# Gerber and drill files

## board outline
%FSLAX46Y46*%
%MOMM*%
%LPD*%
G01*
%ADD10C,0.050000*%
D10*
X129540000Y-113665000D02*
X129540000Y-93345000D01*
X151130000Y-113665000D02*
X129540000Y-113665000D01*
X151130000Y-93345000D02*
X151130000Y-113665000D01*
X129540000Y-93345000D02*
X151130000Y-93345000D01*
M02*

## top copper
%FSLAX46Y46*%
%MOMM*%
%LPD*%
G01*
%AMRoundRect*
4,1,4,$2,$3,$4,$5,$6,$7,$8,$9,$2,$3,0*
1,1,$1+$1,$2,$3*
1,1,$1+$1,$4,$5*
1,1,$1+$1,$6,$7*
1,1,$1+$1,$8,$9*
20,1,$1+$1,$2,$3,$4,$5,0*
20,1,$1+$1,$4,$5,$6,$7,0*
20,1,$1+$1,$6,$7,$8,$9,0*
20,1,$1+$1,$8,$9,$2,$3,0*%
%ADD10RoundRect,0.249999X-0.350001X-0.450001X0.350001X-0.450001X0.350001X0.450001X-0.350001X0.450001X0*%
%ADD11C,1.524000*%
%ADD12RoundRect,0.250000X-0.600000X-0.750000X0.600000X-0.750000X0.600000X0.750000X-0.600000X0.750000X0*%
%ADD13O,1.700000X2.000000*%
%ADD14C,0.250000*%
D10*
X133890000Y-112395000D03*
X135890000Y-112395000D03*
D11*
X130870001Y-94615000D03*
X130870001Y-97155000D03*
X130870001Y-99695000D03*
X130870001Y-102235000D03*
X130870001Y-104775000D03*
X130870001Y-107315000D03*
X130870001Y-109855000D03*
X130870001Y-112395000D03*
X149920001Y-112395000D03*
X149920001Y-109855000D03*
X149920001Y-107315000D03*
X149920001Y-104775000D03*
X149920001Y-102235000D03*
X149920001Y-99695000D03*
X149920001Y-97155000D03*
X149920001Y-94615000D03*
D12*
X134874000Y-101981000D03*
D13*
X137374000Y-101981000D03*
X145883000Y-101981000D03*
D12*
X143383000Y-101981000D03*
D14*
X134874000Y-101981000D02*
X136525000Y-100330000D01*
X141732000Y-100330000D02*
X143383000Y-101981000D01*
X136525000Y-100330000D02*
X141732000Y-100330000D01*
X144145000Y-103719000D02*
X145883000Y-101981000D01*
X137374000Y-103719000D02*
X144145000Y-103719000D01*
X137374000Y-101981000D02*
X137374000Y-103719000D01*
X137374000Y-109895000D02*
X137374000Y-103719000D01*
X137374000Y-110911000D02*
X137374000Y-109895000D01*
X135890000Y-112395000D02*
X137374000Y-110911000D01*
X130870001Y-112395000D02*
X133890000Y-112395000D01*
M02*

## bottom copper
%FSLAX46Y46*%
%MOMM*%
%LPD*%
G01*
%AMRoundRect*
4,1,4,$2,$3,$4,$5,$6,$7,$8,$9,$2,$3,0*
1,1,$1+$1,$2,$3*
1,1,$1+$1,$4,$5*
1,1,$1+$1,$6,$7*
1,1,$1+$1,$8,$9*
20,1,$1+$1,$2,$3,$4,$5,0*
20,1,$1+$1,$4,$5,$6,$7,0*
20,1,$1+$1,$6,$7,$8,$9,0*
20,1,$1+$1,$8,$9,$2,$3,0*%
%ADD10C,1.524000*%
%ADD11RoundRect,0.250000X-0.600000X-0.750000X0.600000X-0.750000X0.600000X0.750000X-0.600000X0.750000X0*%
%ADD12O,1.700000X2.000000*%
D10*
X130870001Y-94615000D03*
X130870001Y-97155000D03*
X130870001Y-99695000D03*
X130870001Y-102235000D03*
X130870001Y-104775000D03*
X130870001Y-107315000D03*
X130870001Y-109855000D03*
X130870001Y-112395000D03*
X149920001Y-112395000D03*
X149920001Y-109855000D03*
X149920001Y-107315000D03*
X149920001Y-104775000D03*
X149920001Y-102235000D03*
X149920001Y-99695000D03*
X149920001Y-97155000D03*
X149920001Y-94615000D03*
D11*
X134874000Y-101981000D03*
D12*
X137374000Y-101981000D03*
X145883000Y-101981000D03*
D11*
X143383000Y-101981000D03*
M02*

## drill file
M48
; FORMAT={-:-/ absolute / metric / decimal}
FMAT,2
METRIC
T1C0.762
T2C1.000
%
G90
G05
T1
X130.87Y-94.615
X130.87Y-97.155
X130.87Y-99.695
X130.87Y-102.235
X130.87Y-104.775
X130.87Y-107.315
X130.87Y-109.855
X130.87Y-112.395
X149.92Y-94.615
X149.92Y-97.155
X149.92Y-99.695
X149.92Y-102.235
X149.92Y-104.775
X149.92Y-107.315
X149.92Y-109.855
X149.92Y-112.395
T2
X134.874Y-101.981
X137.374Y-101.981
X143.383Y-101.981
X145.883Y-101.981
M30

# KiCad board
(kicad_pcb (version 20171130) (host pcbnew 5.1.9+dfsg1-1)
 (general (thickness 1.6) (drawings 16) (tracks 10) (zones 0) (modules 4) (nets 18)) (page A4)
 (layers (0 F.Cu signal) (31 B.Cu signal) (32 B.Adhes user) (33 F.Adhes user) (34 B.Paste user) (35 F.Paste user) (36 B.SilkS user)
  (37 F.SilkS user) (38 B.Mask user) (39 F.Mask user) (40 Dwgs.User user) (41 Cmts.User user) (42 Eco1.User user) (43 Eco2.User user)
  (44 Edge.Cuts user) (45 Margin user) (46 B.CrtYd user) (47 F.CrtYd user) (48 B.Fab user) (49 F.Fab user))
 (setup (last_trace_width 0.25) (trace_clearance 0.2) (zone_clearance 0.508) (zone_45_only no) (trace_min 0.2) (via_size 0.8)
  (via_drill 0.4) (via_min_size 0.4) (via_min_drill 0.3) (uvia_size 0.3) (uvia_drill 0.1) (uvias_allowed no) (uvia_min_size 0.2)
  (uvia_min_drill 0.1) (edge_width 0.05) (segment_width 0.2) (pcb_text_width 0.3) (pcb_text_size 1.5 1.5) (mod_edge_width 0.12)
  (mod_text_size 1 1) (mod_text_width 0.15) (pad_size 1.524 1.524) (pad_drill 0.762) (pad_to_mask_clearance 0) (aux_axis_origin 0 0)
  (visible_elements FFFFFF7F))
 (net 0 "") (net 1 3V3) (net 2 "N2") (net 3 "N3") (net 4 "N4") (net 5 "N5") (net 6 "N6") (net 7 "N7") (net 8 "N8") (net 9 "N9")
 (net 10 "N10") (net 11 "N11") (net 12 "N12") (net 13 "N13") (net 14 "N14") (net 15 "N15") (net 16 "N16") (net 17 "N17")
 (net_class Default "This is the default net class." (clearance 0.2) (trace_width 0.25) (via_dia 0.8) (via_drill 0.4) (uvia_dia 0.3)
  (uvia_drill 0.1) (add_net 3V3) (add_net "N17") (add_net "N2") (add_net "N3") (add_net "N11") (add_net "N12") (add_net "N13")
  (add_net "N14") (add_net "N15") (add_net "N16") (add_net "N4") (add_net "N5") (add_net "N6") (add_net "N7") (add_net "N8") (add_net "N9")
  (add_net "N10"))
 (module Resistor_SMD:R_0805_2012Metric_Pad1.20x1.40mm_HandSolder (layer F.Cu) (at 134.89 112.395)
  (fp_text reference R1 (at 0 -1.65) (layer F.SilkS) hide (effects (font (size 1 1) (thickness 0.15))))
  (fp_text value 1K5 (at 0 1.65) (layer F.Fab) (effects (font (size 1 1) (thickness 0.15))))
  (pad 1 smd roundrect (at -1 0) (size 1.2 1.4) (layers F.Cu F.Paste F.Mask) (roundrect_rratio 0.2083325) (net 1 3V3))
  (pad 2 smd roundrect (at 1 0) (size 1.2 1.4) (layers F.Cu F.Paste F.Mask) (roundrect_rratio 0.2083325) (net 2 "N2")))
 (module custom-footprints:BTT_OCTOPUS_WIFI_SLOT (layer F.Cu) (at 143.570001 94.615)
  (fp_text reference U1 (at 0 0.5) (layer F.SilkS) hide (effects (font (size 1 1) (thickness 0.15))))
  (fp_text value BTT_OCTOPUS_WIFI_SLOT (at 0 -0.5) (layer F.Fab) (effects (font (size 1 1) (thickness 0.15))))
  (pad 1 thru_hole circle (at -12.7 0) (size 1.524 1.524) (drill 0.762) (layers *.Cu *.Mask) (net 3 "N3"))
  (pad 2 thru_hole circle (at -12.7 2.54) (size 1.524 1.524) (drill 0.762) (layers *.Cu *.Mask) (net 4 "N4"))
  (pad 3 thru_hole circle (at -12.7 5.08) (size 1.524 1.524) (drill 0.762) (layers *.Cu *.Mask) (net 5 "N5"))
  (pad 4 thru_hole circle (at -12.7 7.62) (size 1.524 1.524) (drill 0.762) (layers *.Cu *.Mask) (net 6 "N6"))
  (pad 5 thru_hole circle (at -12.7 10.16) (size 1.524 1.524) (drill 0.762) (layers *.Cu *.Mask) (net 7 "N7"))
  (pad 6 thru_hole circle (at -12.7 12.7) (size 1.524 1.524) (drill 0.762) (layers *.Cu *.Mask) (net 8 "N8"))
  (pad 7 thru_hole circle (at -12.7 15.24) (size 1.524 1.524) (drill 0.762) (layers *.Cu *.Mask) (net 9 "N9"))
  (pad 8 thru_hole circle (at -12.7 17.78) (size 1.524 1.524) (drill 0.762) (layers *.Cu *.Mask) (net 1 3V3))
  (pad 9 thru_hole circle (at 6.35 17.78) (size 1.524 1.524) (drill 0.762) (layers *.Cu *.Mask) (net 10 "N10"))
  (pad 10 thru_hole circle (at 6.35 15.24) (size 1.524 1.524) (drill 0.762) (layers *.Cu *.Mask) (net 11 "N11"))
  (pad 11 thru_hole circle (at 6.35 12.7) (size 1.524 1.524) (drill 0.762) (layers *.Cu *.Mask) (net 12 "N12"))
  (pad 12 thru_hole circle (at 6.35 10.16) (size 1.524 1.524) (drill 0.762) (layers *.Cu *.Mask) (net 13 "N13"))
  (pad 13 thru_hole circle (at 6.35 7.62) (size 1.524 1.524) (drill 0.762) (layers *.Cu *.Mask) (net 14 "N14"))
  (pad 14 thru_hole circle (at 6.35 5.08) (size 1.524 1.524) (drill 0.762) (layers *.Cu *.Mask) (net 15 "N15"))
  (pad 15 thru_hole circle (at 6.35 2.54) (size 1.524 1.524) (drill 0.762) (layers *.Cu *.Mask) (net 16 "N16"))
  (pad 16 thru_hole circle (at 6.35 0) (size 1.524 1.524) (drill 0.762) (layers *.Cu *.Mask)))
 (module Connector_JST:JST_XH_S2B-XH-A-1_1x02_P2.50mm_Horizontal (layer B.Cu) (at 134.874 101.981)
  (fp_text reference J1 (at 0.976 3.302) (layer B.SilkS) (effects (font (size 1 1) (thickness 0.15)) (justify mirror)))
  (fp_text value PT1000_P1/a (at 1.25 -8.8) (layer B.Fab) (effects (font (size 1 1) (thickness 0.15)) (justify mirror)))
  (pad 1 thru_hole roundrect (at 0 0) (size 1.7 2) (drill 1) (layers *.Cu *.Mask) (roundrect_rratio 0.1470588235294118) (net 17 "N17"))
  (pad 2 thru_hole oval (at 2.5 0) (size 1.7 2) (drill 1) (layers *.Cu *.Mask) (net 2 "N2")))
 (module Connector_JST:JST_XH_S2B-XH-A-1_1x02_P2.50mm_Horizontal (layer B.Cu) (at 143.383 101.981)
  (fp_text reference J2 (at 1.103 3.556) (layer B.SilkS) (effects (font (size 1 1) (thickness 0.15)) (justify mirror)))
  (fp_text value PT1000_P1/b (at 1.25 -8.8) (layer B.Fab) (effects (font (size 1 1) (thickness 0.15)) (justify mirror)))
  (pad 2 thru_hole oval (at 2.5 0) (size 1.7 2) (drill 1) (layers *.Cu *.Mask) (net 2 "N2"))
  (pad 1 thru_hole roundrect (at 0 0) (size 1.7 2) (drill 1) (layers *.Cu *.Mask) (roundrect_rratio 0.1470588235294118) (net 17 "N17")))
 (gr_line (start 129.54 113.665) (end 129.54 93.345) (layer Edge.Cuts) (width 0.05))
 (gr_line (start 151.13 113.665) (end 129.54 113.665) (layer Edge.Cuts) (width 0.05))
 (gr_line (start 151.13 93.345) (end 151.13 113.665) (layer Edge.Cuts) (width 0.05))
 (gr_line (start 129.54 93.345) (end 151.13 93.345) (layer Edge.Cuts) (width 0.05))
 (segment (start 134.874 101.981) (end 136.525 100.33) (width 0.25) (layer F.Cu) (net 17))
 (segment (start 141.732 100.33) (end 143.383 101.981) (width 0.25) (layer F.Cu) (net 17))
 (segment (start 136.525 100.33) (end 141.732 100.33) (width 0.25) (layer F.Cu) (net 17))
 (segment (start 144.145 103.719) (end 145.883 101.981) (width 0.25) (layer F.Cu) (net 2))
 (segment (start 137.374 103.719) (end 144.145 103.719) (width 0.25) (layer F.Cu) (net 2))
 (segment (start 137.374 101.981) (end 137.374 103.719) (width 0.25) (layer F.Cu) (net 2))
 (segment (start 137.374 109.895) (end 137.374 103.719) (width 0.25) (layer F.Cu) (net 2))
 (segment (start 137.374 110.911) (end 137.374 109.895) (width 0.25) (layer F.Cu) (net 2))
 (segment (start 135.89 112.395) (end 137.374 110.911) (width 0.25) (layer F.Cu) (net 2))
 (segment (start 130.870001 112.395) (end 133.89 112.395) (width 0.25) (layer F.Cu) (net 1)))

